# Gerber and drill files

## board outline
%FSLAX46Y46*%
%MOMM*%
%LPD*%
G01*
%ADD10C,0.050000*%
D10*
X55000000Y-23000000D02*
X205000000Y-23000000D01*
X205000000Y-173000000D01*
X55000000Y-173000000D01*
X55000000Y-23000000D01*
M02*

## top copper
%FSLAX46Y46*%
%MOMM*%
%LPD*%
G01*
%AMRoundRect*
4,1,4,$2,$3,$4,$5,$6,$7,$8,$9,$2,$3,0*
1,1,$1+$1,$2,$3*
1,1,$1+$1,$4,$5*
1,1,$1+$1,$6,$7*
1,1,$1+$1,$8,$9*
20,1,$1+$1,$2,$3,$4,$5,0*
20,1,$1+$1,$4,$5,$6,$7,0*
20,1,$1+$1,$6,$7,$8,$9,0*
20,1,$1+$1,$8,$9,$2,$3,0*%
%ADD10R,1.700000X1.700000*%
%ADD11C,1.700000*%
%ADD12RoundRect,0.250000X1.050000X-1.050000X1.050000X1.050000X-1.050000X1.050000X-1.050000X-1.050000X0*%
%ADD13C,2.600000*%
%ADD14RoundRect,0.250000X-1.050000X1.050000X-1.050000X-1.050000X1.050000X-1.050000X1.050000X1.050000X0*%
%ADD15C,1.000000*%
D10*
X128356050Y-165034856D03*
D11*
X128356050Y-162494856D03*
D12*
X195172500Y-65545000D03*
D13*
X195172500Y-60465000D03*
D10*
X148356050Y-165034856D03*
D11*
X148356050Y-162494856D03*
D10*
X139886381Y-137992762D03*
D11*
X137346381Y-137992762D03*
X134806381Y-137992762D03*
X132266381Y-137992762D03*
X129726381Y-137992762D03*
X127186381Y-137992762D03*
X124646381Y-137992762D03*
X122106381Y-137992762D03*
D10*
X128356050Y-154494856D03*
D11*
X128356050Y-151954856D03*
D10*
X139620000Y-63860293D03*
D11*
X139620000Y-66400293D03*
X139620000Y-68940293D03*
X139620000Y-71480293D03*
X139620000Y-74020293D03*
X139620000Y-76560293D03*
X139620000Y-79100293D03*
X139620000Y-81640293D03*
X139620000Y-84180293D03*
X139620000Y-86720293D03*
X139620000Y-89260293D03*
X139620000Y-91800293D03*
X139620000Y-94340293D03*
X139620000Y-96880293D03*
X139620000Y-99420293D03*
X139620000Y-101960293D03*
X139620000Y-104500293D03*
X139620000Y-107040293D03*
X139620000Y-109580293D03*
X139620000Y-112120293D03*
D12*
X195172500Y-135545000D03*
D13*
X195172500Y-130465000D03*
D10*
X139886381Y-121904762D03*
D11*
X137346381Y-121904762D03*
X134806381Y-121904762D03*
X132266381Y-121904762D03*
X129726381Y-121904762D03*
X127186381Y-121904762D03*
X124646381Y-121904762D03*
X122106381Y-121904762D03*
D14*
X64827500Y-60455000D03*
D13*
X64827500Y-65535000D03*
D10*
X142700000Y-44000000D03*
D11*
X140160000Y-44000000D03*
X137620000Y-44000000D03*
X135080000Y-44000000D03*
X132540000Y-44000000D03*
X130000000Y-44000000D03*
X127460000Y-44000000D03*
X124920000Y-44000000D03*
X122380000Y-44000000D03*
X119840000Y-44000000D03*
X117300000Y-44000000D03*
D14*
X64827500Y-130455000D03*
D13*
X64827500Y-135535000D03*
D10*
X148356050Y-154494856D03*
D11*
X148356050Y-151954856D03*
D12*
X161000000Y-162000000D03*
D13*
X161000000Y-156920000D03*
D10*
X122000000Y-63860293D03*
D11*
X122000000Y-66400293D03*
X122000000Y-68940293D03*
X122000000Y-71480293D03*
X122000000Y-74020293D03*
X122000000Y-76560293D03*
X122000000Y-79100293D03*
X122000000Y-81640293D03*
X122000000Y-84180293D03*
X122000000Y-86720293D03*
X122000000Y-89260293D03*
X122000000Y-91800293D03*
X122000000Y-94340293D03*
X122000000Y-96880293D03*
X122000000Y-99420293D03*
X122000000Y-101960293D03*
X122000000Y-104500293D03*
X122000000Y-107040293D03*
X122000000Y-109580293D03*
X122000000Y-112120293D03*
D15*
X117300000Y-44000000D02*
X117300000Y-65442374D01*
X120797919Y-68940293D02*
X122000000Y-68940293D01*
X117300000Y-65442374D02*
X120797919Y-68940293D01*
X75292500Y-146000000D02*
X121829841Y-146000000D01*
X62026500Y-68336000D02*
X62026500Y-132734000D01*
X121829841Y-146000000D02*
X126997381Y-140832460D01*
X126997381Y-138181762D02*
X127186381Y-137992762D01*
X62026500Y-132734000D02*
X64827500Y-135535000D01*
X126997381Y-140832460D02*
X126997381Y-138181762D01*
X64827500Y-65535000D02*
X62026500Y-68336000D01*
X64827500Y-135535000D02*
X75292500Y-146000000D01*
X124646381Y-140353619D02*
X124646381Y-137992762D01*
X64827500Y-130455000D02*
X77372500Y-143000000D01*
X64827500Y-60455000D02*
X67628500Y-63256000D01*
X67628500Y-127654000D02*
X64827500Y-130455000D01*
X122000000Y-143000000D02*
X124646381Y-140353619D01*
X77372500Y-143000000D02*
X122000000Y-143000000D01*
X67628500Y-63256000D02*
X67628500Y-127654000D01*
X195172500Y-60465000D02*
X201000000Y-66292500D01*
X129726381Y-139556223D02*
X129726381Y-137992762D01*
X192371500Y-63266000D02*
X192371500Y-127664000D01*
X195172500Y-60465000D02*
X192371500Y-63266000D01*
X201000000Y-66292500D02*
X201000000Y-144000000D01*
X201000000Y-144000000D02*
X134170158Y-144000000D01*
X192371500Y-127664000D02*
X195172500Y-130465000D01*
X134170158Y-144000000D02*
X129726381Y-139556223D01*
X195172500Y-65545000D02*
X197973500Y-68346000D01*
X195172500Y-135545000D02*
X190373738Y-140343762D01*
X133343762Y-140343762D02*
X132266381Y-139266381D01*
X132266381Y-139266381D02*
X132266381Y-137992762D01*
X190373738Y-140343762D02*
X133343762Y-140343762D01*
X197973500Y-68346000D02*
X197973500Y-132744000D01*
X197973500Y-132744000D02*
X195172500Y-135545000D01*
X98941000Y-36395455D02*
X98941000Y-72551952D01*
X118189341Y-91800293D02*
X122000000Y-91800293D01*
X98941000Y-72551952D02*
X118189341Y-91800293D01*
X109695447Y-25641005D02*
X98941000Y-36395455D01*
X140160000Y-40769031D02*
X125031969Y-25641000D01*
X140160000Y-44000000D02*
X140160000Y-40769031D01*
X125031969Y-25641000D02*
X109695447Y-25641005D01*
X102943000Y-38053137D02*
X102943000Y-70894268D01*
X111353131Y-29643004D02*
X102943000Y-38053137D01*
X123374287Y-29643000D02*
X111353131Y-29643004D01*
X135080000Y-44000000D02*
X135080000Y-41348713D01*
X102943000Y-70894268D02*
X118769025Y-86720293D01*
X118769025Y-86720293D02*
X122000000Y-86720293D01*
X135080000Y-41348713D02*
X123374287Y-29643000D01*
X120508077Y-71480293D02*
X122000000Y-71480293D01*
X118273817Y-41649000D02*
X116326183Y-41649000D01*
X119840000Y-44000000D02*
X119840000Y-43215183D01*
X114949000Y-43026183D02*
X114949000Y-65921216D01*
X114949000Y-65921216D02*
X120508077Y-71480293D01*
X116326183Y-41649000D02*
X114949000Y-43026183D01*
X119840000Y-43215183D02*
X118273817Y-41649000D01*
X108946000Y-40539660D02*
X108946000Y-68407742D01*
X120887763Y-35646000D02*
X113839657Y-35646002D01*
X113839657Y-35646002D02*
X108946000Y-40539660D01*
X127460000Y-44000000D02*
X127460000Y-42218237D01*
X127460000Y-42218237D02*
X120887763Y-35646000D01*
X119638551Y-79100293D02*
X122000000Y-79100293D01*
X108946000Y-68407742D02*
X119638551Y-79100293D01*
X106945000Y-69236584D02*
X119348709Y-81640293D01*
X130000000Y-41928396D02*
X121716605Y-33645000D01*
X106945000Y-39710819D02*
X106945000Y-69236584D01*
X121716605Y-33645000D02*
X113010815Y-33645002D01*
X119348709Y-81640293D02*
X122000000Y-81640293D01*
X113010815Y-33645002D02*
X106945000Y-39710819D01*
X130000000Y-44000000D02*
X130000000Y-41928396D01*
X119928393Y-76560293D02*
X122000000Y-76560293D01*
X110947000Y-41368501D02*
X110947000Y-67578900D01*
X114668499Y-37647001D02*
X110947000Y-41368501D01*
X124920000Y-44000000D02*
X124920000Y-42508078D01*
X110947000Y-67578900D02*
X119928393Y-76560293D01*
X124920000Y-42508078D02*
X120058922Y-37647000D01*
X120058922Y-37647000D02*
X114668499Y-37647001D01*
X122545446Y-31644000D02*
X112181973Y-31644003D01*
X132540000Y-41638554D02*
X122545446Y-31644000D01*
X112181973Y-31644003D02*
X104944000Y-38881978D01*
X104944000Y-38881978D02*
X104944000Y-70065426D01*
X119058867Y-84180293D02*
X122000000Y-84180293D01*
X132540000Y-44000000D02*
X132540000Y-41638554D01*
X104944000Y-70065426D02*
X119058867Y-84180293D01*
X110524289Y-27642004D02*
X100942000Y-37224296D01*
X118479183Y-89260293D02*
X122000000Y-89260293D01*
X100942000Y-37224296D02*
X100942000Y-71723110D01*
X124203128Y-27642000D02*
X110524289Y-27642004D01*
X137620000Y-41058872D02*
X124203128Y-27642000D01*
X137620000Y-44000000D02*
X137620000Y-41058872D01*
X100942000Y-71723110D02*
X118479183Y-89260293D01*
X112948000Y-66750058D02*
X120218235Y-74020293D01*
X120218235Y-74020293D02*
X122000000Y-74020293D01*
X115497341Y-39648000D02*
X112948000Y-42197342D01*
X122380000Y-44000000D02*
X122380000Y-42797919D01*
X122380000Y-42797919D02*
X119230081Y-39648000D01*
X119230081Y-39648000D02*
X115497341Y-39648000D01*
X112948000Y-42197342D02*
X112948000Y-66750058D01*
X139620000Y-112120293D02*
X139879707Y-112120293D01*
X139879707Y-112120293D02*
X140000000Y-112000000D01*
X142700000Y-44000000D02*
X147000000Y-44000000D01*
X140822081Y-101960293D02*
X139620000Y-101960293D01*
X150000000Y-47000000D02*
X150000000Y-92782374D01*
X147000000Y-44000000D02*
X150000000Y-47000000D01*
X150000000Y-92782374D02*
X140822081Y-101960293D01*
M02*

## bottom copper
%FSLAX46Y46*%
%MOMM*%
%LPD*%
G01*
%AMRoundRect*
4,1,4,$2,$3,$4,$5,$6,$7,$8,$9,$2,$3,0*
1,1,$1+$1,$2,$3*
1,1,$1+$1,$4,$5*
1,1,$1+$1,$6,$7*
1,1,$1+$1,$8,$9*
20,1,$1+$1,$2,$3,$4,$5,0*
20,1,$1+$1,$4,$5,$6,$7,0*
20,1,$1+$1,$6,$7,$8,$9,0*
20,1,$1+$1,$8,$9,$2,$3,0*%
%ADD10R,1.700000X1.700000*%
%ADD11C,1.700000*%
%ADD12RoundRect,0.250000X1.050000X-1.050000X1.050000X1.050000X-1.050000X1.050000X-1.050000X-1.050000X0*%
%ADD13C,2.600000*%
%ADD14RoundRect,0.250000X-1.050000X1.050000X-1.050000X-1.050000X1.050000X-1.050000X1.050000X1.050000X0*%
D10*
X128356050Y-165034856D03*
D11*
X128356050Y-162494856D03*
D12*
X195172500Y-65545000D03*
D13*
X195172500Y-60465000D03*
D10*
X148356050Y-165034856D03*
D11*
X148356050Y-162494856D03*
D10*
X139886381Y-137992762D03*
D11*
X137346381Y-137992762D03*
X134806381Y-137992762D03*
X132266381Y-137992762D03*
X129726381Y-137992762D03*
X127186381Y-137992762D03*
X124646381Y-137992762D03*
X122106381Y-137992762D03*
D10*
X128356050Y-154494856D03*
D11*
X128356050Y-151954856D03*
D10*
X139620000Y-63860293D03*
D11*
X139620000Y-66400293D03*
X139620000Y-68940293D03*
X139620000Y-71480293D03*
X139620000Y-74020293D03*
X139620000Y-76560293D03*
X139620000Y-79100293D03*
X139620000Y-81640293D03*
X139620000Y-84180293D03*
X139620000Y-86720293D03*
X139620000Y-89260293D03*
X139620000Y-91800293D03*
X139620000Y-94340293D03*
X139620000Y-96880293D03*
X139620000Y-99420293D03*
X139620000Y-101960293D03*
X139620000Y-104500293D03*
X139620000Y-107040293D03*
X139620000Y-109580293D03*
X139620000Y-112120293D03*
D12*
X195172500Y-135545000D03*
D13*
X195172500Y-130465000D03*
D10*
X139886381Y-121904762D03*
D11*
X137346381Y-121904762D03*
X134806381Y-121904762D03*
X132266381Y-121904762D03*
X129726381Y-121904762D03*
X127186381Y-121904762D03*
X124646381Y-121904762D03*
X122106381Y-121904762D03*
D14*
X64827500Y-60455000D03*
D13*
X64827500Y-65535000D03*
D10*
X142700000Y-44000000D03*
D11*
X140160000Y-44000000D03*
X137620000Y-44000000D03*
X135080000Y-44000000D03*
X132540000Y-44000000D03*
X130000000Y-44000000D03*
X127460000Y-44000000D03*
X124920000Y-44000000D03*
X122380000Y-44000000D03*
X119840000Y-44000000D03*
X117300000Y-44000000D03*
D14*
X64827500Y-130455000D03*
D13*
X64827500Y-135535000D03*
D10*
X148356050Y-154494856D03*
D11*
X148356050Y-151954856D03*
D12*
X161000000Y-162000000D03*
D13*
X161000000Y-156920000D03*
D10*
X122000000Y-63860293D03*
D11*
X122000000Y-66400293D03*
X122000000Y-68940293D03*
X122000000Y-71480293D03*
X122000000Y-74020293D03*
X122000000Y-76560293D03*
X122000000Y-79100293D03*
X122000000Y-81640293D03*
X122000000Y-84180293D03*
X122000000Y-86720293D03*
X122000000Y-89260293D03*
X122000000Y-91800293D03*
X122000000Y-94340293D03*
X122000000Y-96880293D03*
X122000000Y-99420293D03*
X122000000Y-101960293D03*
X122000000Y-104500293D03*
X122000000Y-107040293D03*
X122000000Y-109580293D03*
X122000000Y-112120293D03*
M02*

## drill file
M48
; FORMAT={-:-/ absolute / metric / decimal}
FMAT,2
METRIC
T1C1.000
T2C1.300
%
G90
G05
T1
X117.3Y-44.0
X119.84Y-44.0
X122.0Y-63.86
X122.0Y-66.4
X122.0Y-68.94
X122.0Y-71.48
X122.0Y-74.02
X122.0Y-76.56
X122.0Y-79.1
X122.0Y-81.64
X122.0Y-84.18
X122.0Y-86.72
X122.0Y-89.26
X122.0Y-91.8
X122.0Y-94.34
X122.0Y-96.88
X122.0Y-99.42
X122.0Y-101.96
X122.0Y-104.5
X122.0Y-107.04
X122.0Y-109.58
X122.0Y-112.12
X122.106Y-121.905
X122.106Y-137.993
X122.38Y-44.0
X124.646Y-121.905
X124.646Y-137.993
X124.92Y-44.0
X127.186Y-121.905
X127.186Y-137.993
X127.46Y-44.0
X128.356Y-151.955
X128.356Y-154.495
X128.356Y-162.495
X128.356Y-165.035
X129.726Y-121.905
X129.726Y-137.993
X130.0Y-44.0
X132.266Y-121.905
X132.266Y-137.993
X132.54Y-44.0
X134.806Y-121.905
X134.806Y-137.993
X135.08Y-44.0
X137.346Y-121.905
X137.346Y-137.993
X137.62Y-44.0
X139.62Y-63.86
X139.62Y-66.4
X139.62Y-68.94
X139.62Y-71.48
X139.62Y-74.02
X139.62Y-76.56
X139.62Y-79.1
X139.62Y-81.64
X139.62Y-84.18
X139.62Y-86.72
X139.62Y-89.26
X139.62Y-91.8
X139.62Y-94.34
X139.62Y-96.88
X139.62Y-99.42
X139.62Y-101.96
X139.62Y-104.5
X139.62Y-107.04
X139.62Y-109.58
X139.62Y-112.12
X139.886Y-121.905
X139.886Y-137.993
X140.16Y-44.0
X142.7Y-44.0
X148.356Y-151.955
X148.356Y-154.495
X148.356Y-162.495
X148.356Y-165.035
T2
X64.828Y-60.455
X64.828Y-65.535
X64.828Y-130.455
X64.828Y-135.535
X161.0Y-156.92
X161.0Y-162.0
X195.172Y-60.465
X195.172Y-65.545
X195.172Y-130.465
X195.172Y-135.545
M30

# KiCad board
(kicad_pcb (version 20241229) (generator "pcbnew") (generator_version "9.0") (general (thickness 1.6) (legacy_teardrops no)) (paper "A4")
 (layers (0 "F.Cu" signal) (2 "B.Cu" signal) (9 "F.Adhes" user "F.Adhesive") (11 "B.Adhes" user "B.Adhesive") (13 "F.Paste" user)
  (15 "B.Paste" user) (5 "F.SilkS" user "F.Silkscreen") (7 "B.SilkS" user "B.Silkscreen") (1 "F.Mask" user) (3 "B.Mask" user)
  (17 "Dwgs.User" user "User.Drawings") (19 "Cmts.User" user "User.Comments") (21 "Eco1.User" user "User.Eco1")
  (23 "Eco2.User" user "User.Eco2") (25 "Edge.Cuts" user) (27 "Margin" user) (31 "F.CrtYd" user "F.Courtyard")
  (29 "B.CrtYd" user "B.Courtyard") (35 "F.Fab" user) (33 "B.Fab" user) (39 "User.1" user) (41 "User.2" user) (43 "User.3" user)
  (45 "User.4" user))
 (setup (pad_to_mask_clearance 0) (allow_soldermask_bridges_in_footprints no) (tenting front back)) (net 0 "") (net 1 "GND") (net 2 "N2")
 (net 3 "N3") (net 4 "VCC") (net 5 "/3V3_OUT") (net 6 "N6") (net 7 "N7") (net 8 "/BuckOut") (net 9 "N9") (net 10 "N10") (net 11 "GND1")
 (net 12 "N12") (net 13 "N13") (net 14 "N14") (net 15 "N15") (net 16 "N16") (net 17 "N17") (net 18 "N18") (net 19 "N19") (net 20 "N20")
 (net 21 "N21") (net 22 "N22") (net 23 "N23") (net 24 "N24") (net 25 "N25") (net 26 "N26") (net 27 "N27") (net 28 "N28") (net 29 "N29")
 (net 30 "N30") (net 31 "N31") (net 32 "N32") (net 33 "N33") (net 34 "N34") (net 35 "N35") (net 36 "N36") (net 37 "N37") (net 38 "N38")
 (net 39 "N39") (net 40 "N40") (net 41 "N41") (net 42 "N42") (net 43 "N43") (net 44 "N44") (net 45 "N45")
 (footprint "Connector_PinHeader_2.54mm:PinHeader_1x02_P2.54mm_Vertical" (layer "F.Cu") (at 128.35605 165.034856 180)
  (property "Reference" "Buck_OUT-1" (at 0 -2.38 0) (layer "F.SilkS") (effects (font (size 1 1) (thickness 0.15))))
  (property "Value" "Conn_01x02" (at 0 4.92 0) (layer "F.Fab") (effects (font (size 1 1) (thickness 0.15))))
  (pad "1" thru_hole rect (at 0 0 180) (size 1.7 1.7) (drill 1) (layers "*.Cu" "*.Mask") (remove_unused_layers no) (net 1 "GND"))
  (pad "2" thru_hole circle (at 0 2.54 180) (size 1.7 1.7) (drill 1) (layers "*.Cu" "*.Mask") (remove_unused_layers no) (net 1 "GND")))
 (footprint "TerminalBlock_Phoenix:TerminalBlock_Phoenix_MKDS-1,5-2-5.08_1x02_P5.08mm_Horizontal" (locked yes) (layer "F.Cu")
  (at 195.1725 65.545 90)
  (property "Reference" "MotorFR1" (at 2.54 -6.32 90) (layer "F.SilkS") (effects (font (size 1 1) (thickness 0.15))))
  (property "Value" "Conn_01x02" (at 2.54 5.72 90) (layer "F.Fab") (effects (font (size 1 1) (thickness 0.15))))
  (pad "1" thru_hole roundrect (at 0 0 90) (size 2.6 2.6) (drill 1.3) (layers "*.Cu" "*.Mask") (remove_unused_layers no)
   (roundrect_rratio 0.096154) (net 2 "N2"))
  (pad "2" thru_hole circle (at 5.08 0 90) (size 2.6 2.6) (drill 1.3) (layers "*.Cu" "*.Mask") (remove_unused_layers no) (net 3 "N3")))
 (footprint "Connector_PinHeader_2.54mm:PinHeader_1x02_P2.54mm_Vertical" (layer "F.Cu") (at 148.35605 165.034856 180)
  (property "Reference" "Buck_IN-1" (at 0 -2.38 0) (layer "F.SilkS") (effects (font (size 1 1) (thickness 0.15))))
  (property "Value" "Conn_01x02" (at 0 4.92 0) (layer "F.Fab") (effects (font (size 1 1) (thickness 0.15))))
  (pad "1" thru_hole rect (at 0 0 180) (size 1.7 1.7) (drill 1) (layers "*.Cu" "*.Mask") (remove_unused_layers no) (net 1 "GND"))
  (pad "2" thru_hole circle (at 0 2.54 180) (size 1.7 1.7) (drill 1) (layers "*.Cu" "*.Mask") (remove_unused_layers no) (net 1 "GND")))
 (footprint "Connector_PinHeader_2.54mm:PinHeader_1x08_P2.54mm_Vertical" (layer "F.Cu") (at 139.886381 137.992762 -90)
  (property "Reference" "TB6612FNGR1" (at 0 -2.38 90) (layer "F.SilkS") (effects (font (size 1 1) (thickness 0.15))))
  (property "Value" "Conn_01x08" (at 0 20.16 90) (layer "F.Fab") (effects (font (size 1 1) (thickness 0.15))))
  (pad "1" thru_hole rect (at 0 0 270) (size 1.7 1.7) (drill 1) (layers "*.Cu" "*.Mask") (remove_unused_layers no) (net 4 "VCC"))
  (pad "2" thru_hole circle (at 0 2.54 270) (size 1.7 1.7) (drill 1) (layers "*.Cu" "*.Mask") (remove_unused_layers no) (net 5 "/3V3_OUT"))
  (pad "3" thru_hole circle (at 0 5.08 270) (size 1.7 1.7) (drill 1) (layers "*.Cu" "*.Mask") (remove_unused_layers no) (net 1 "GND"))
  (pad "4" thru_hole circle (at 0 7.62 270) (size 1.7 1.7) (drill 1) (layers "*.Cu" "*.Mask") (remove_unused_layers no) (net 2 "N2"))
  (pad "5" thru_hole circle (at 0 10.16 270) (size 1.7 1.7) (drill 1) (layers "*.Cu" "*.Mask") (remove_unused_layers no) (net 3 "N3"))
  (pad "6" thru_hole circle (at 0 12.7 270) (size 1.7 1.7) (drill 1) (layers "*.Cu" "*.Mask") (remove_unused_layers no) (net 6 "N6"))
  (pad "7" thru_hole circle (at 0 15.24 270) (size 1.7 1.7) (drill 1) (layers "*.Cu" "*.Mask") (remove_unused_layers no) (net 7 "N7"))
  (pad "8" thru_hole circle (at 0 17.78 270) (size 1.7 1.7) (drill 1) (layers "*.Cu" "*.Mask") (remove_unused_layers no) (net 1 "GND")))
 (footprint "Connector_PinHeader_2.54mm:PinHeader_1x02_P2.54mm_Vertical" (layer "F.Cu") (at 128.35605 154.494856 180)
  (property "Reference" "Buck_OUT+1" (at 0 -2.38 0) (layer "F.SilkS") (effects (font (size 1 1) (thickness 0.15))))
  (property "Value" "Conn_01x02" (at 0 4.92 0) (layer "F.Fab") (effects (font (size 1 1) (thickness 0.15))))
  (pad "1" thru_hole rect (at 0 0 180) (size 1.7 1.7) (drill 1) (layers "*.Cu" "*.Mask") (remove_unused_layers no) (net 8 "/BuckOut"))
  (pad "2" thru_hole circle (at 0 2.54 180) (size 1.7 1.7) (drill 1) (layers "*.Cu" "*.Mask") (remove_unused_layers no) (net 8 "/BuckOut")))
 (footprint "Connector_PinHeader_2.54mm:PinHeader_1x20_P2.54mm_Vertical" (layer "F.Cu") (at 139.62 63.860293)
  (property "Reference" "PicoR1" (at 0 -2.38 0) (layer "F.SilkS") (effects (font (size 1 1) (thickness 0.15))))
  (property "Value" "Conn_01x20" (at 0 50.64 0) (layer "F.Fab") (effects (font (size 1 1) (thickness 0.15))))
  (pad "1" thru_hole rect (at 0 0) (size 1.7 1.7) (drill 1) (layers "*.Cu" "*.Mask") (remove_unused_layers no) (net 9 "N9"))
  (pad "2" thru_hole circle (at 0 2.54) (size 1.7 1.7) (drill 1) (layers "*.Cu" "*.Mask") (remove_unused_layers no) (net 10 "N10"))
  (pad "3" thru_hole circle (at 0 5.08) (size 1.7 1.7) (drill 1) (layers "*.Cu" "*.Mask") (remove_unused_layers no) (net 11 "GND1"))
  (pad "4" thru_hole circle (at 0 7.62) (size 1.7 1.7) (drill 1) (layers "*.Cu" "*.Mask") (remove_unused_layers no) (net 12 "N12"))
  (pad "5" thru_hole circle (at 0 10.16) (size 1.7 1.7) (drill 1) (layers "*.Cu" "*.Mask") (remove_unused_layers no) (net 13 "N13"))
  (pad "6" thru_hole circle (at 0 12.7) (size 1.7 1.7) (drill 1) (layers "*.Cu" "*.Mask") (remove_unused_layers no) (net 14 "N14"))
  (pad "7" thru_hole circle (at 0 15.24) (size 1.7 1.7) (drill 1) (layers "*.Cu" "*.Mask") (remove_unused_layers no) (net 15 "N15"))
  (pad "8" thru_hole circle (at 0 17.78) (size 1.7 1.7) (drill 1) (layers "*.Cu" "*.Mask") (remove_unused_layers no) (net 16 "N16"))
  (pad "9" thru_hole circle (at 0 20.32) (size 1.7 1.7) (drill 1) (layers "*.Cu" "*.Mask") (remove_unused_layers no) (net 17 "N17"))
  (pad "10" thru_hole circle (at 0 22.86) (size 1.7 1.7) (drill 1) (layers "*.Cu" "*.Mask") (remove_unused_layers no) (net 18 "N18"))
  (pad "11" thru_hole circle (at 0 25.4) (size 1.7 1.7) (drill 1) (layers "*.Cu" "*.Mask") (remove_unused_layers no) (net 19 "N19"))
  (pad "12" thru_hole circle (at 0 27.94) (size 1.7 1.7) (drill 1) (layers "*.Cu" "*.Mask") (remove_unused_layers no) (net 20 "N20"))
  (pad "13" thru_hole circle (at 0 30.48) (size 1.7 1.7) (drill 1) (layers "*.Cu" "*.Mask") (remove_unused_layers no) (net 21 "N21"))
  (pad "14" thru_hole circle (at 0 33.02) (size 1.7 1.7) (drill 1) (layers "*.Cu" "*.Mask") (remove_unused_layers no) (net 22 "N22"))
  (pad "15" thru_hole circle (at 0 35.56) (size 1.7 1.7) (drill 1) (layers "*.Cu" "*.Mask") (remove_unused_layers no) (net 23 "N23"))
  (pad "16" thru_hole circle (at 0 38.1) (size 1.7 1.7) (drill 1) (layers "*.Cu" "*.Mask") (remove_unused_layers no) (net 5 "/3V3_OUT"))
  (pad "17" thru_hole circle (at 0 40.64) (size 1.7 1.7) (drill 1) (layers "*.Cu" "*.Mask") (remove_unused_layers no) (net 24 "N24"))
  (pad "18" thru_hole circle (at 0 43.18) (size 1.7 1.7) (drill 1) (layers "*.Cu" "*.Mask") (remove_unused_layers no) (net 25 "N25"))
  (pad "19" thru_hole circle (at 0 45.72) (size 1.7 1.7) (drill 1) (layers "*.Cu" "*.Mask") (remove_unused_layers no) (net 8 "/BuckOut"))
  (pad "20" thru_hole circle (at 0 48.26) (size 1.7 1.7) (drill 1) (layers "*.Cu" "*.Mask") (remove_unused_layers no) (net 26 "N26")))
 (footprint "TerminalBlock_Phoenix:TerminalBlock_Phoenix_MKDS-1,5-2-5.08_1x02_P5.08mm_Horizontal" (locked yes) (layer "F.Cu")
  (at 195.1725 135.545 90)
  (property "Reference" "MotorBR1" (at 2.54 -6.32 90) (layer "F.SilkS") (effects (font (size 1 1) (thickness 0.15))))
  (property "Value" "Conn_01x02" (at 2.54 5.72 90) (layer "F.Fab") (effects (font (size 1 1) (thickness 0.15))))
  (pad "1" thru_hole roundrect (at 0 0 90) (size 2.6 2.6) (drill 1.3) (layers "*.Cu" "*.Mask") (remove_unused_layers no)
   (roundrect_rratio 0.096154) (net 2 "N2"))
  (pad "2" thru_hole circle (at 5.08 0 90) (size 2.6 2.6) (drill 1.3) (layers "*.Cu" "*.Mask") (remove_unused_layers no) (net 3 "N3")))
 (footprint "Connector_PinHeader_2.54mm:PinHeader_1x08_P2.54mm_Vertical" (layer "F.Cu") (at 139.886381 121.904762 -90)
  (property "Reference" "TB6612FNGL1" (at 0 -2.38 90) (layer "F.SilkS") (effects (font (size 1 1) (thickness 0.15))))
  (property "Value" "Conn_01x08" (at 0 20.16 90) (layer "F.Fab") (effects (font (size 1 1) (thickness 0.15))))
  (pad "1" thru_hole rect (at 0 0 270) (size 1.7 1.7) (drill 1) (layers "*.Cu" "*.Mask") (remove_unused_layers no) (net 11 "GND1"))
  (pad "2" thru_hole circle (at 0 2.54 270) (size 1.7 1.7) (drill 1) (layers "*.Cu" "*.Mask") (remove_unused_layers no) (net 15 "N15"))
  (pad "3" thru_hole circle (at 0 5.08 270) (size 1.7 1.7) (drill 1) (layers "*.Cu" "*.Mask") (remove_unused_layers no) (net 14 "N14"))
  (pad "4" thru_hole circle (at 0 7.62 270) (size 1.7 1.7) (drill 1) (layers "*.Cu" "*.Mask") (remove_unused_layers no) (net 13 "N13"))
  (pad "5" thru_hole circle (at 0 10.16 270) (size 1.7 1.7) (drill 1) (layers "*.Cu" "*.Mask") (remove_unused_layers no) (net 5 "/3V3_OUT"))
  (pad "6" thru_hole circle (at 0 12.7 270) (size 1.7 1.7) (drill 1) (layers "*.Cu" "*.Mask") (remove_unused_layers no) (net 12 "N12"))
  (pad "7" thru_hole circle (at 0 15.24 270) (size 1.7 1.7) (drill 1) (layers "*.Cu" "*.Mask") (remove_unused_layers no) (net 10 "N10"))
  (pad "8" thru_hole circle (at 0 17.78 270) (size 1.7 1.7) (drill 1) (layers "*.Cu" "*.Mask") (remove_unused_layers no) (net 9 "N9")))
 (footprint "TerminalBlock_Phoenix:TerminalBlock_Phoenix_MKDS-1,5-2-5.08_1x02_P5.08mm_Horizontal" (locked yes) (layer "F.Cu")
  (at 64.8275 60.455 -90)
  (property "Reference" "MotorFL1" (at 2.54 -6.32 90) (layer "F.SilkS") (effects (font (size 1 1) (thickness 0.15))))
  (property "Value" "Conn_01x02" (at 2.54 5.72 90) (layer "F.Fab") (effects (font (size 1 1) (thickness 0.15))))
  (pad "1" thru_hole roundrect (at 0 0 270) (size 2.6 2.6) (drill 1.3) (layers "*.Cu" "*.Mask") (remove_unused_layers no)
   (roundrect_rratio 0.096154) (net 7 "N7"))
  (pad "2" thru_hole circle (at 5.08 0 270) (size 2.6 2.6) (drill 1.3) (layers "*.Cu" "*.Mask") (remove_unused_layers no) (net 6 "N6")))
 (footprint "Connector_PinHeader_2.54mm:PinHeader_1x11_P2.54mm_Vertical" (layer "F.Cu") (at 142.7 44 -90)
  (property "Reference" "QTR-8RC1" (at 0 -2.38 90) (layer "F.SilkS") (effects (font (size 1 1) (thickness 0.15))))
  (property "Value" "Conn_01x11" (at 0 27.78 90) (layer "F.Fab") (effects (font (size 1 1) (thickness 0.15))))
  (pad "1" thru_hole rect (at 0 0 270) (size 1.7 1.7) (drill 1) (layers "*.Cu" "*.Mask") (remove_unused_layers no) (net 5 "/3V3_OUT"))
  (pad "2" thru_hole circle (at 0 2.54 270) (size 1.7 1.7) (drill 1) (layers "*.Cu" "*.Mask") (remove_unused_layers no) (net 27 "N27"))
  (pad "3" thru_hole circle (at 0 5.08 270) (size 1.7 1.7) (drill 1) (layers "*.Cu" "*.Mask") (remove_unused_layers no) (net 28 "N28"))
  (pad "4" thru_hole circle (at 0 7.62 270) (size 1.7 1.7) (drill 1) (layers "*.Cu" "*.Mask") (remove_unused_layers no) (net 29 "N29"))
  (pad "5" thru_hole circle (at 0 10.16 270) (size 1.7 1.7) (drill 1) (layers "*.Cu" "*.Mask") (remove_unused_layers no) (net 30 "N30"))
  (pad "6" thru_hole circle (at 0 12.7 270) (size 1.7 1.7) (drill 1) (layers "*.Cu" "*.Mask") (remove_unused_layers no) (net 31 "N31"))
  (pad "7" thru_hole circle (at 0 15.24 270) (size 1.7 1.7) (drill 1) (layers "*.Cu" "*.Mask") (remove_unused_layers no) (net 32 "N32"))
  (pad "8" thru_hole circle (at 0 17.78 270) (size 1.7 1.7) (drill 1) (layers "*.Cu" "*.Mask") (remove_unused_layers no) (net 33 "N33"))
  (pad "9" thru_hole circle (at 0 20.32 270) (size 1.7 1.7) (drill 1) (layers "*.Cu" "*.Mask") (remove_unused_layers no) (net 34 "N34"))
  (pad "10" thru_hole circle (at 0 22.86 270) (size 1.7 1.7) (drill 1) (layers "*.Cu" "*.Mask") (remove_unused_layers no) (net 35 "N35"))
  (pad "11" thru_hole circle (at 0 25.4 270) (size 1.7 1.7) (drill 1) (layers "*.Cu" "*.Mask") (remove_unused_layers no) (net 1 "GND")))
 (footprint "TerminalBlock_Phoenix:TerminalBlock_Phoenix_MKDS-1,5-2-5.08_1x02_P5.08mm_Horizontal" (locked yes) (layer "F.Cu")
  (at 64.8275 130.455 -90)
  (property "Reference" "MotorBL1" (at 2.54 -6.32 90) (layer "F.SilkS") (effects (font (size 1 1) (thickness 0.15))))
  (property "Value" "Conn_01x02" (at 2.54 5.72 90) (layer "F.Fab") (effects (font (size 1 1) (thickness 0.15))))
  (pad "1" thru_hole roundrect (at 0 0 270) (size 2.6 2.6) (drill 1.3) (layers "*.Cu" "*.Mask") (remove_unused_layers no)
   (roundrect_rratio 0.096154) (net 7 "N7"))
  (pad "2" thru_hole circle (at 5.08 0 270) (size 2.6 2.6) (drill 1.3) (layers "*.Cu" "*.Mask") (remove_unused_layers no) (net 6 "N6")))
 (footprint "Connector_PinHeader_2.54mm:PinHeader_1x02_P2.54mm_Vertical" (layer "F.Cu") (at 148.35605 154.494856 180)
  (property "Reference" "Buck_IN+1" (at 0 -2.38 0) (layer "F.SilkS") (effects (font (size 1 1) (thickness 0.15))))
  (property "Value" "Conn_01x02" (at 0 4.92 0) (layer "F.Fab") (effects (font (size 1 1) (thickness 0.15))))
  (pad "1" thru_hole rect (at 0 0 180) (size 1.7 1.7) (drill 1) (layers "*.Cu" "*.Mask") (remove_unused_layers no) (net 4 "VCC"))
  (pad "2" thru_hole circle (at 0 2.54 180) (size 1.7 1.7) (drill 1) (layers "*.Cu" "*.Mask") (remove_unused_layers no) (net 4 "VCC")))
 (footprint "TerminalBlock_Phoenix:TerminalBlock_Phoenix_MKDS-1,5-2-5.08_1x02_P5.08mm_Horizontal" (layer "F.Cu") (at 161 162 90)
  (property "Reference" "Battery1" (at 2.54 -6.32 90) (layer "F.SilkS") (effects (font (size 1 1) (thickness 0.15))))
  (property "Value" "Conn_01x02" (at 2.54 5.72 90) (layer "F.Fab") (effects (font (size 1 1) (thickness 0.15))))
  (pad "1" thru_hole roundrect (at 0 0 90) (size 2.6 2.6) (drill 1.3) (layers "*.Cu" "*.Mask") (remove_unused_layers no)
   (roundrect_rratio 0.096154) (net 1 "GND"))
  (pad "2" thru_hole circle (at 5.08 0 90) (size 2.6 2.6) (drill 1.3) (layers "*.Cu" "*.Mask") (remove_unused_layers no) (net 4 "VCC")))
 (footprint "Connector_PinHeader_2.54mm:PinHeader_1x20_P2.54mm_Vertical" (layer "F.Cu") (at 122 63.860293)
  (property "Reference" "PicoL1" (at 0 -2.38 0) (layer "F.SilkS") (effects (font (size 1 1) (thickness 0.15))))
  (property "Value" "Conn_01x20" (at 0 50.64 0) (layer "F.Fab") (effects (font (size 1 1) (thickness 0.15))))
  (pad "1" thru_hole rect (at 0 0) (size 1.7 1.7) (drill 1) (layers "*.Cu" "*.Mask") (remove_unused_layers no) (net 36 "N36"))
  (pad "2" thru_hole circle (at 0 2.54) (size 1.7 1.7) (drill 1) (layers "*.Cu" "*.Mask") (remove_unused_layers no) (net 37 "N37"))
  (pad "3" thru_hole circle (at 0 5.08) (size 1.7 1.7) (drill 1) (layers "*.Cu" "*.Mask") (remove_unused_layers no) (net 1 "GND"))
  (pad "4" thru_hole circle (at 0 7.62) (size 1.7 1.7) (drill 1) (layers "*.Cu" "*.Mask") (remove_unused_layers no) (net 35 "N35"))
  (pad "5" thru_hole circle (at 0 10.16) (size 1.7 1.7) (drill 1) (layers "*.Cu" "*.Mask") (remove_unused_layers no) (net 34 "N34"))
  (pad "6" thru_hole circle (at 0 12.7) (size 1.7 1.7) (drill 1) (layers "*.Cu" "*.Mask") (remove_unused_layers no) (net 33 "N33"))
  (pad "7" thru_hole circle (at 0 15.24) (size 1.7 1.7) (drill 1) (layers "*.Cu" "*.Mask") (remove_unused_layers no) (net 32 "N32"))
  (pad "8" thru_hole circle (at 0 17.78) (size 1.7 1.7) (drill 1) (layers "*.Cu" "*.Mask") (remove_unused_layers no) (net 31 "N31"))
  (pad "9" thru_hole circle (at 0 20.32) (size 1.7 1.7) (drill 1) (layers "*.Cu" "*.Mask") (remove_unused_layers no) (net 30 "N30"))
  (pad "10" thru_hole circle (at 0 22.86) (size 1.7 1.7) (drill 1) (layers "*.Cu" "*.Mask") (remove_unused_layers no) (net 29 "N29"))
  (pad "11" thru_hole circle (at 0 25.4) (size 1.7 1.7) (drill 1) (layers "*.Cu" "*.Mask") (remove_unused_layers no) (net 28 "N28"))
  (pad "12" thru_hole circle (at 0 27.94) (size 1.7 1.7) (drill 1) (layers "*.Cu" "*.Mask") (remove_unused_layers no) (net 27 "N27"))
  (pad "13" thru_hole circle (at 0 30.48) (size 1.7 1.7) (drill 1) (layers "*.Cu" "*.Mask") (remove_unused_layers no) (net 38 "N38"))
  (pad "14" thru_hole circle (at 0 33.02) (size 1.7 1.7) (drill 1) (layers "*.Cu" "*.Mask") (remove_unused_layers no) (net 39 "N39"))
  (pad "15" thru_hole circle (at 0 35.56) (size 1.7 1.7) (drill 1) (layers "*.Cu" "*.Mask") (remove_unused_layers no) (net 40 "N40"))
  (pad "16" thru_hole circle (at 0 38.1) (size 1.7 1.7) (drill 1) (layers "*.Cu" "*.Mask") (remove_unused_layers no) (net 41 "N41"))
  (pad "17" thru_hole circle (at 0 40.64) (size 1.7 1.7) (drill 1) (layers "*.Cu" "*.Mask") (remove_unused_layers no) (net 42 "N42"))
  (pad "18" thru_hole circle (at 0 43.18) (size 1.7 1.7) (drill 1) (layers "*.Cu" "*.Mask") (remove_unused_layers no) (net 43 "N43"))
  (pad "19" thru_hole circle (at 0 45.72) (size 1.7 1.7) (drill 1) (layers "*.Cu" "*.Mask") (remove_unused_layers no) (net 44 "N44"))
  (pad "20" thru_hole circle (at 0 48.26) (size 1.7 1.7) (drill 1) (layers "*.Cu" "*.Mask") (remove_unused_layers no) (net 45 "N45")))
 (gr_rect (start 55 23) (end 205 173) (stroke (width 0.05) (type default)) (fill no) (layer "Edge.Cuts"))
 (segment (start 117.3 44) (end 117.3 65.442374) (width 1) (layer "F.Cu") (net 1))
 (segment (start 120.797919 68.940293) (end 122 68.940293) (width 1) (layer "F.Cu") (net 1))
 (segment (start 117.3 65.442374) (end 120.797919 68.940293) (width 1) (layer "F.Cu") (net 1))
 (segment (start 75.2925 146) (end 121.829841 146) (width 1) (layer "F.Cu") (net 6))
 (segment (start 62.0265 68.336) (end 62.0265 132.734) (width 1) (layer "F.Cu") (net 6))
 (segment (start 121.829841 146) (end 126.997381 140.83246) (width 1) (layer "F.Cu") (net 6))
 (segment (start 126.997381 138.181762) (end 127.186381 137.992762) (width 1) (layer "F.Cu") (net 6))
 (segment (start 62.0265 132.734) (end 64.8275 135.535) (width 1) (layer "F.Cu") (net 6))
 (segment (start 126.997381 140.83246) (end 126.997381 138.181762) (width 1) (layer "F.Cu") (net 6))
 (segment (start 64.8275 65.535) (end 62.0265 68.336) (width 1) (layer "F.Cu") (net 6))
 (segment (start 64.8275 135.535) (end 75.2925 146) (width 1) (layer "F.Cu") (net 6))
 (segment (start 124.646381 140.353619) (end 124.646381 137.992762) (width 1) (layer "F.Cu") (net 7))
 (segment (start 64.8275 130.455) (end 77.3725 143) (width 1) (layer "F.Cu") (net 7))
 (segment (start 64.8275 60.455) (end 67.6285 63.256) (width 1) (layer "F.Cu") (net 7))
 (segment (start 67.6285 127.654) (end 64.8275 130.455) (width 1) (layer "F.Cu") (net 7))
 (segment (start 122 143) (end 124.646381 140.353619) (width 1) (layer "F.Cu") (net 7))
 (segment (start 77.3725 143) (end 122 143) (width 1) (layer "F.Cu") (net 7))
 (segment (start 67.6285 63.256) (end 67.6285 127.654) (width 1) (layer "F.Cu") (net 7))
 (segment (start 195.1725 60.465) (end 201 66.2925) (width 1) (layer "F.Cu") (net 3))
 (segment (start 129.726381 139.556223) (end 129.726381 137.992762) (width 1) (layer "F.Cu") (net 3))
 (segment (start 192.3715 63.266) (end 192.3715 127.664) (width 1) (layer "F.Cu") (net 3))
 (segment (start 195.1725 60.465) (end 192.3715 63.266) (width 1) (layer "F.Cu") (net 3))
 (segment (start 201 66.2925) (end 201 144) (width 1) (layer "F.Cu") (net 3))
 (segment (start 201 144) (end 134.170158 144) (width 1) (layer "F.Cu") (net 3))
 (segment (start 192.3715 127.664) (end 195.1725 130.465) (width 1) (layer "F.Cu") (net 3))
 (segment (start 134.170158 144) (end 129.726381 139.556223) (width 1) (layer "F.Cu") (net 3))
 (segment (start 195.1725 65.545) (end 197.9735 68.346) (width 1) (layer "F.Cu") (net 2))
 (segment (start 195.1725 135.545) (end 190.373738 140.343762) (width 1) (layer "F.Cu") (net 2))
 (segment (start 133.343762 140.343762) (end 132.266381 139.266381) (width 1) (layer "F.Cu") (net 2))
 (segment (start 132.266381 139.266381) (end 132.266381 137.992762) (width 1) (layer "F.Cu") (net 2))
 (segment (start 190.373738 140.343762) (end 133.343762 140.343762) (width 1) (layer "F.Cu") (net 2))
 (segment (start 197.9735 68.346) (end 197.9735 132.744) (width 1) (layer "F.Cu") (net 2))
 (segment (start 197.9735 132.744) (end 195.1725 135.545) (width 1) (layer "F.Cu") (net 2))
 (segment (start 98.941 36.395455) (end 98.941 72.551952) (width 1) (layer "F.Cu") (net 27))
 (segment (start 118.189341 91.800293) (end 122 91.800293) (width 1) (layer "F.Cu") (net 27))
 (segment (start 98.941 72.551952) (end 118.189341 91.800293) (width 1) (layer "F.Cu") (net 27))
 (segment (start 109.695447 25.641005) (end 98.941 36.395455) (width 1) (layer "F.Cu") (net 27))
 (segment (start 140.16 40.769031) (end 125.031969 25.641) (width 1) (layer "F.Cu") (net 27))
 (segment (start 140.16 44) (end 140.16 40.769031) (width 1) (layer "F.Cu") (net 27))
 (segment (start 125.031969 25.641) (end 109.695447 25.641005) (width 1) (layer "F.Cu") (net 27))
 (segment (start 102.943 38.053137) (end 102.943 70.894268) (width 1) (layer "F.Cu") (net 29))
 (segment (start 111.353131 29.643004) (end 102.943 38.053137) (width 1) (layer "F.Cu") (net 29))
 (segment (start 123.374287 29.643) (end 111.353131 29.643004) (width 1) (layer "F.Cu") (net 29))
 (segment (start 135.08 44) (end 135.08 41.348713) (width 1) (layer "F.Cu") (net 29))
 (segment (start 102.943 70.894268) (end 118.769025 86.720293) (width 1) (layer "F.Cu") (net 29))
 (segment (start 118.769025 86.720293) (end 122 86.720293) (width 1) (layer "F.Cu") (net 29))
 (segment (start 135.08 41.348713) (end 123.374287 29.643) (width 1) (layer "F.Cu") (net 29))
 (segment (start 120.508077 71.480293) (end 122 71.480293) (width 1) (layer "F.Cu") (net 35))
 (segment (start 118.273817 41.649) (end 116.326183 41.649) (width 1) (layer "F.Cu") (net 35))
 (segment (start 119.84 44) (end 119.84 43.215183) (width 1) (layer "F.Cu") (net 35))
 (segment (start 114.949 43.026183) (end 114.949 65.921216) (width 1) (layer "F.Cu") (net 35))
 (segment (start 114.949 65.921216) (end 120.508077 71.480293) (width 1) (layer "F.Cu") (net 35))
 (segment (start 116.326183 41.649) (end 114.949 43.026183) (width 1) (layer "F.Cu") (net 35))
 (segment (start 119.84 43.215183) (end 118.273817 41.649) (width 1) (layer "F.Cu") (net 35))
 (segment (start 108.946 40.53966) (end 108.946 68.407742) (width 1) (layer "F.Cu") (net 32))
 (segment (start 120.887763 35.646) (end 113.839657 35.646002) (width 1) (layer "F.Cu") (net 32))
 (segment (start 113.839657 35.646002) (end 108.946 40.53966) (width 1) (layer "F.Cu") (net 32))
 (segment (start 127.46 44) (end 127.46 42.218237) (width 1) (layer "F.Cu") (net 32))
 (segment (start 127.46 42.218237) (end 120.887763 35.646) (width 1) (layer "F.Cu") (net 32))
 (segment (start 119.638551 79.100293) (end 122 79.100293) (width 1) (layer "F.Cu") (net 32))
 (segment (start 108.946 68.407742) (end 119.638551 79.100293) (width 1) (layer "F.Cu") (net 32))
 (segment (start 106.945 69.236584) (end 119.348709 81.640293) (width 1) (layer "F.Cu") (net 31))
 (segment (start 130 41.928396) (end 121.716605 33.645) (width 1) (layer "F.Cu") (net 31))
 (segment (start 106.945 39.710819) (end 106.945 69.236584) (width 1) (layer "F.Cu") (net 31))
 (segment (start 121.716605 33.645) (end 113.010815 33.645002) (width 1) (layer "F.Cu") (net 31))
 (segment (start 119.348709 81.640293) (end 122 81.640293) (width 1) (layer "F.Cu") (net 31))
 (segment (start 113.010815 33.645002) (end 106.945 39.710819) (width 1) (layer "F.Cu") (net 31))
 (segment (start 130 44) (end 130 41.928396) (width 1) (layer "F.Cu") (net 31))
 (segment (start 119.928393 76.560293) (end 122 76.560293) (width 1) (layer "F.Cu") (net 33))
 (segment (start 110.947 41.368501) (end 110.947 67.5789) (width 1) (layer "F.Cu") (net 33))
 (segment (start 114.668499 37.647001) (end 110.947 41.368501) (width 1) (layer "F.Cu") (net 33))
 (segment (start 124.92 44) (end 124.92 42.508078) (width 1) (layer "F.Cu") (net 33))
 (segment (start 110.947 67.5789) (end 119.928393 76.560293) (width 1) (layer "F.Cu") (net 33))
 (segment (start 124.92 42.508078) (end 120.058922 37.647) (width 1) (layer "F.Cu") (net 33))
 (segment (start 120.058922 37.647) (end 114.668499 37.647001) (width 1) (layer "F.Cu") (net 33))
 (segment (start 122.545446 31.644) (end 112.181973 31.644003) (width 1) (layer "F.Cu") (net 30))
 (segment (start 132.54 41.638554) (end 122.545446 31.644) (width 1) (layer "F.Cu") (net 30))
 (segment (start 112.181973 31.644003) (end 104.944 38.881978) (width 1) (layer "F.Cu") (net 30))
 (segment (start 104.944 38.881978) (end 104.944 70.065426) (width 1) (layer "F.Cu") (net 30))
 (segment (start 119.058867 84.180293) (end 122 84.180293) (width 1) (layer "F.Cu") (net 30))
 (segment (start 132.54 44) (end 132.54 41.638554) (width 1) (layer "F.Cu") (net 30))
 (segment (start 104.944 70.065426) (end 119.058867 84.180293) (width 1) (layer "F.Cu") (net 30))
 (segment (start 110.524289 27.642004) (end 100.942 37.224296) (width 1) (layer "F.Cu") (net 28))
 (segment (start 118.479183 89.260293) (end 122 89.260293) (width 1) (layer "F.Cu") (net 28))
 (segment (start 100.942 37.224296) (end 100.942 71.72311) (width 1) (layer "F.Cu") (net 28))
 (segment (start 124.203128 27.642) (end 110.524289 27.642004) (width 1) (layer "F.Cu") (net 28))
 (segment (start 137.62 41.058872) (end 124.203128 27.642) (width 1) (layer "F.Cu") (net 28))
 (segment (start 137.62 44) (end 137.62 41.058872) (width 1) (layer "F.Cu") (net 28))
 (segment (start 100.942 71.72311) (end 118.479183 89.260293) (width 1) (layer "F.Cu") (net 28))
 (segment (start 112.948 66.750058) (end 120.218235 74.020293) (width 1) (layer "F.Cu") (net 34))
 (segment (start 120.218235 74.020293) (end 122 74.020293) (width 1) (layer "F.Cu") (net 34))
 (segment (start 115.497341 39.648) (end 112.948 42.197342) (width 1) (layer "F.Cu") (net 34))
 (segment (start 122.38 44) (end 122.38 42.797919) (width 1) (layer "F.Cu") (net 34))
 (segment (start 122.38 42.797919) (end 119.230081 39.648) (width 1) (layer "F.Cu") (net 34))
 (segment (start 119.230081 39.648) (end 115.497341 39.648) (width 1) (layer "F.Cu") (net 34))
 (segment (start 112.948 42.197342) (end 112.948 66.750058) (width 1) (layer "F.Cu") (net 34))
 (segment (start 139.62 112.120293) (end 139.879707 112.120293) (width 1) (layer "F.Cu") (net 26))
 (segment (start 139.879707 112.120293) (end 140 112) (width 1) (layer "F.Cu") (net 26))
 (segment (start 142.7 44) (end 147 44) (width 1) (layer "F.Cu") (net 5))
 (segment (start 140.822081 101.960293) (end 139.62 101.960293) (width 1) (layer "F.Cu") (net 5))
 (segment (start 150 47) (end 150 92.782374) (width 1) (layer "F.Cu") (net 5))
 (segment (start 147 44) (end 150 47) (width 1) (layer "F.Cu") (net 5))
 (segment (start 150 92.782374) (end 140.822081 101.960293) (width 1) (layer "F.Cu") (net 5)))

